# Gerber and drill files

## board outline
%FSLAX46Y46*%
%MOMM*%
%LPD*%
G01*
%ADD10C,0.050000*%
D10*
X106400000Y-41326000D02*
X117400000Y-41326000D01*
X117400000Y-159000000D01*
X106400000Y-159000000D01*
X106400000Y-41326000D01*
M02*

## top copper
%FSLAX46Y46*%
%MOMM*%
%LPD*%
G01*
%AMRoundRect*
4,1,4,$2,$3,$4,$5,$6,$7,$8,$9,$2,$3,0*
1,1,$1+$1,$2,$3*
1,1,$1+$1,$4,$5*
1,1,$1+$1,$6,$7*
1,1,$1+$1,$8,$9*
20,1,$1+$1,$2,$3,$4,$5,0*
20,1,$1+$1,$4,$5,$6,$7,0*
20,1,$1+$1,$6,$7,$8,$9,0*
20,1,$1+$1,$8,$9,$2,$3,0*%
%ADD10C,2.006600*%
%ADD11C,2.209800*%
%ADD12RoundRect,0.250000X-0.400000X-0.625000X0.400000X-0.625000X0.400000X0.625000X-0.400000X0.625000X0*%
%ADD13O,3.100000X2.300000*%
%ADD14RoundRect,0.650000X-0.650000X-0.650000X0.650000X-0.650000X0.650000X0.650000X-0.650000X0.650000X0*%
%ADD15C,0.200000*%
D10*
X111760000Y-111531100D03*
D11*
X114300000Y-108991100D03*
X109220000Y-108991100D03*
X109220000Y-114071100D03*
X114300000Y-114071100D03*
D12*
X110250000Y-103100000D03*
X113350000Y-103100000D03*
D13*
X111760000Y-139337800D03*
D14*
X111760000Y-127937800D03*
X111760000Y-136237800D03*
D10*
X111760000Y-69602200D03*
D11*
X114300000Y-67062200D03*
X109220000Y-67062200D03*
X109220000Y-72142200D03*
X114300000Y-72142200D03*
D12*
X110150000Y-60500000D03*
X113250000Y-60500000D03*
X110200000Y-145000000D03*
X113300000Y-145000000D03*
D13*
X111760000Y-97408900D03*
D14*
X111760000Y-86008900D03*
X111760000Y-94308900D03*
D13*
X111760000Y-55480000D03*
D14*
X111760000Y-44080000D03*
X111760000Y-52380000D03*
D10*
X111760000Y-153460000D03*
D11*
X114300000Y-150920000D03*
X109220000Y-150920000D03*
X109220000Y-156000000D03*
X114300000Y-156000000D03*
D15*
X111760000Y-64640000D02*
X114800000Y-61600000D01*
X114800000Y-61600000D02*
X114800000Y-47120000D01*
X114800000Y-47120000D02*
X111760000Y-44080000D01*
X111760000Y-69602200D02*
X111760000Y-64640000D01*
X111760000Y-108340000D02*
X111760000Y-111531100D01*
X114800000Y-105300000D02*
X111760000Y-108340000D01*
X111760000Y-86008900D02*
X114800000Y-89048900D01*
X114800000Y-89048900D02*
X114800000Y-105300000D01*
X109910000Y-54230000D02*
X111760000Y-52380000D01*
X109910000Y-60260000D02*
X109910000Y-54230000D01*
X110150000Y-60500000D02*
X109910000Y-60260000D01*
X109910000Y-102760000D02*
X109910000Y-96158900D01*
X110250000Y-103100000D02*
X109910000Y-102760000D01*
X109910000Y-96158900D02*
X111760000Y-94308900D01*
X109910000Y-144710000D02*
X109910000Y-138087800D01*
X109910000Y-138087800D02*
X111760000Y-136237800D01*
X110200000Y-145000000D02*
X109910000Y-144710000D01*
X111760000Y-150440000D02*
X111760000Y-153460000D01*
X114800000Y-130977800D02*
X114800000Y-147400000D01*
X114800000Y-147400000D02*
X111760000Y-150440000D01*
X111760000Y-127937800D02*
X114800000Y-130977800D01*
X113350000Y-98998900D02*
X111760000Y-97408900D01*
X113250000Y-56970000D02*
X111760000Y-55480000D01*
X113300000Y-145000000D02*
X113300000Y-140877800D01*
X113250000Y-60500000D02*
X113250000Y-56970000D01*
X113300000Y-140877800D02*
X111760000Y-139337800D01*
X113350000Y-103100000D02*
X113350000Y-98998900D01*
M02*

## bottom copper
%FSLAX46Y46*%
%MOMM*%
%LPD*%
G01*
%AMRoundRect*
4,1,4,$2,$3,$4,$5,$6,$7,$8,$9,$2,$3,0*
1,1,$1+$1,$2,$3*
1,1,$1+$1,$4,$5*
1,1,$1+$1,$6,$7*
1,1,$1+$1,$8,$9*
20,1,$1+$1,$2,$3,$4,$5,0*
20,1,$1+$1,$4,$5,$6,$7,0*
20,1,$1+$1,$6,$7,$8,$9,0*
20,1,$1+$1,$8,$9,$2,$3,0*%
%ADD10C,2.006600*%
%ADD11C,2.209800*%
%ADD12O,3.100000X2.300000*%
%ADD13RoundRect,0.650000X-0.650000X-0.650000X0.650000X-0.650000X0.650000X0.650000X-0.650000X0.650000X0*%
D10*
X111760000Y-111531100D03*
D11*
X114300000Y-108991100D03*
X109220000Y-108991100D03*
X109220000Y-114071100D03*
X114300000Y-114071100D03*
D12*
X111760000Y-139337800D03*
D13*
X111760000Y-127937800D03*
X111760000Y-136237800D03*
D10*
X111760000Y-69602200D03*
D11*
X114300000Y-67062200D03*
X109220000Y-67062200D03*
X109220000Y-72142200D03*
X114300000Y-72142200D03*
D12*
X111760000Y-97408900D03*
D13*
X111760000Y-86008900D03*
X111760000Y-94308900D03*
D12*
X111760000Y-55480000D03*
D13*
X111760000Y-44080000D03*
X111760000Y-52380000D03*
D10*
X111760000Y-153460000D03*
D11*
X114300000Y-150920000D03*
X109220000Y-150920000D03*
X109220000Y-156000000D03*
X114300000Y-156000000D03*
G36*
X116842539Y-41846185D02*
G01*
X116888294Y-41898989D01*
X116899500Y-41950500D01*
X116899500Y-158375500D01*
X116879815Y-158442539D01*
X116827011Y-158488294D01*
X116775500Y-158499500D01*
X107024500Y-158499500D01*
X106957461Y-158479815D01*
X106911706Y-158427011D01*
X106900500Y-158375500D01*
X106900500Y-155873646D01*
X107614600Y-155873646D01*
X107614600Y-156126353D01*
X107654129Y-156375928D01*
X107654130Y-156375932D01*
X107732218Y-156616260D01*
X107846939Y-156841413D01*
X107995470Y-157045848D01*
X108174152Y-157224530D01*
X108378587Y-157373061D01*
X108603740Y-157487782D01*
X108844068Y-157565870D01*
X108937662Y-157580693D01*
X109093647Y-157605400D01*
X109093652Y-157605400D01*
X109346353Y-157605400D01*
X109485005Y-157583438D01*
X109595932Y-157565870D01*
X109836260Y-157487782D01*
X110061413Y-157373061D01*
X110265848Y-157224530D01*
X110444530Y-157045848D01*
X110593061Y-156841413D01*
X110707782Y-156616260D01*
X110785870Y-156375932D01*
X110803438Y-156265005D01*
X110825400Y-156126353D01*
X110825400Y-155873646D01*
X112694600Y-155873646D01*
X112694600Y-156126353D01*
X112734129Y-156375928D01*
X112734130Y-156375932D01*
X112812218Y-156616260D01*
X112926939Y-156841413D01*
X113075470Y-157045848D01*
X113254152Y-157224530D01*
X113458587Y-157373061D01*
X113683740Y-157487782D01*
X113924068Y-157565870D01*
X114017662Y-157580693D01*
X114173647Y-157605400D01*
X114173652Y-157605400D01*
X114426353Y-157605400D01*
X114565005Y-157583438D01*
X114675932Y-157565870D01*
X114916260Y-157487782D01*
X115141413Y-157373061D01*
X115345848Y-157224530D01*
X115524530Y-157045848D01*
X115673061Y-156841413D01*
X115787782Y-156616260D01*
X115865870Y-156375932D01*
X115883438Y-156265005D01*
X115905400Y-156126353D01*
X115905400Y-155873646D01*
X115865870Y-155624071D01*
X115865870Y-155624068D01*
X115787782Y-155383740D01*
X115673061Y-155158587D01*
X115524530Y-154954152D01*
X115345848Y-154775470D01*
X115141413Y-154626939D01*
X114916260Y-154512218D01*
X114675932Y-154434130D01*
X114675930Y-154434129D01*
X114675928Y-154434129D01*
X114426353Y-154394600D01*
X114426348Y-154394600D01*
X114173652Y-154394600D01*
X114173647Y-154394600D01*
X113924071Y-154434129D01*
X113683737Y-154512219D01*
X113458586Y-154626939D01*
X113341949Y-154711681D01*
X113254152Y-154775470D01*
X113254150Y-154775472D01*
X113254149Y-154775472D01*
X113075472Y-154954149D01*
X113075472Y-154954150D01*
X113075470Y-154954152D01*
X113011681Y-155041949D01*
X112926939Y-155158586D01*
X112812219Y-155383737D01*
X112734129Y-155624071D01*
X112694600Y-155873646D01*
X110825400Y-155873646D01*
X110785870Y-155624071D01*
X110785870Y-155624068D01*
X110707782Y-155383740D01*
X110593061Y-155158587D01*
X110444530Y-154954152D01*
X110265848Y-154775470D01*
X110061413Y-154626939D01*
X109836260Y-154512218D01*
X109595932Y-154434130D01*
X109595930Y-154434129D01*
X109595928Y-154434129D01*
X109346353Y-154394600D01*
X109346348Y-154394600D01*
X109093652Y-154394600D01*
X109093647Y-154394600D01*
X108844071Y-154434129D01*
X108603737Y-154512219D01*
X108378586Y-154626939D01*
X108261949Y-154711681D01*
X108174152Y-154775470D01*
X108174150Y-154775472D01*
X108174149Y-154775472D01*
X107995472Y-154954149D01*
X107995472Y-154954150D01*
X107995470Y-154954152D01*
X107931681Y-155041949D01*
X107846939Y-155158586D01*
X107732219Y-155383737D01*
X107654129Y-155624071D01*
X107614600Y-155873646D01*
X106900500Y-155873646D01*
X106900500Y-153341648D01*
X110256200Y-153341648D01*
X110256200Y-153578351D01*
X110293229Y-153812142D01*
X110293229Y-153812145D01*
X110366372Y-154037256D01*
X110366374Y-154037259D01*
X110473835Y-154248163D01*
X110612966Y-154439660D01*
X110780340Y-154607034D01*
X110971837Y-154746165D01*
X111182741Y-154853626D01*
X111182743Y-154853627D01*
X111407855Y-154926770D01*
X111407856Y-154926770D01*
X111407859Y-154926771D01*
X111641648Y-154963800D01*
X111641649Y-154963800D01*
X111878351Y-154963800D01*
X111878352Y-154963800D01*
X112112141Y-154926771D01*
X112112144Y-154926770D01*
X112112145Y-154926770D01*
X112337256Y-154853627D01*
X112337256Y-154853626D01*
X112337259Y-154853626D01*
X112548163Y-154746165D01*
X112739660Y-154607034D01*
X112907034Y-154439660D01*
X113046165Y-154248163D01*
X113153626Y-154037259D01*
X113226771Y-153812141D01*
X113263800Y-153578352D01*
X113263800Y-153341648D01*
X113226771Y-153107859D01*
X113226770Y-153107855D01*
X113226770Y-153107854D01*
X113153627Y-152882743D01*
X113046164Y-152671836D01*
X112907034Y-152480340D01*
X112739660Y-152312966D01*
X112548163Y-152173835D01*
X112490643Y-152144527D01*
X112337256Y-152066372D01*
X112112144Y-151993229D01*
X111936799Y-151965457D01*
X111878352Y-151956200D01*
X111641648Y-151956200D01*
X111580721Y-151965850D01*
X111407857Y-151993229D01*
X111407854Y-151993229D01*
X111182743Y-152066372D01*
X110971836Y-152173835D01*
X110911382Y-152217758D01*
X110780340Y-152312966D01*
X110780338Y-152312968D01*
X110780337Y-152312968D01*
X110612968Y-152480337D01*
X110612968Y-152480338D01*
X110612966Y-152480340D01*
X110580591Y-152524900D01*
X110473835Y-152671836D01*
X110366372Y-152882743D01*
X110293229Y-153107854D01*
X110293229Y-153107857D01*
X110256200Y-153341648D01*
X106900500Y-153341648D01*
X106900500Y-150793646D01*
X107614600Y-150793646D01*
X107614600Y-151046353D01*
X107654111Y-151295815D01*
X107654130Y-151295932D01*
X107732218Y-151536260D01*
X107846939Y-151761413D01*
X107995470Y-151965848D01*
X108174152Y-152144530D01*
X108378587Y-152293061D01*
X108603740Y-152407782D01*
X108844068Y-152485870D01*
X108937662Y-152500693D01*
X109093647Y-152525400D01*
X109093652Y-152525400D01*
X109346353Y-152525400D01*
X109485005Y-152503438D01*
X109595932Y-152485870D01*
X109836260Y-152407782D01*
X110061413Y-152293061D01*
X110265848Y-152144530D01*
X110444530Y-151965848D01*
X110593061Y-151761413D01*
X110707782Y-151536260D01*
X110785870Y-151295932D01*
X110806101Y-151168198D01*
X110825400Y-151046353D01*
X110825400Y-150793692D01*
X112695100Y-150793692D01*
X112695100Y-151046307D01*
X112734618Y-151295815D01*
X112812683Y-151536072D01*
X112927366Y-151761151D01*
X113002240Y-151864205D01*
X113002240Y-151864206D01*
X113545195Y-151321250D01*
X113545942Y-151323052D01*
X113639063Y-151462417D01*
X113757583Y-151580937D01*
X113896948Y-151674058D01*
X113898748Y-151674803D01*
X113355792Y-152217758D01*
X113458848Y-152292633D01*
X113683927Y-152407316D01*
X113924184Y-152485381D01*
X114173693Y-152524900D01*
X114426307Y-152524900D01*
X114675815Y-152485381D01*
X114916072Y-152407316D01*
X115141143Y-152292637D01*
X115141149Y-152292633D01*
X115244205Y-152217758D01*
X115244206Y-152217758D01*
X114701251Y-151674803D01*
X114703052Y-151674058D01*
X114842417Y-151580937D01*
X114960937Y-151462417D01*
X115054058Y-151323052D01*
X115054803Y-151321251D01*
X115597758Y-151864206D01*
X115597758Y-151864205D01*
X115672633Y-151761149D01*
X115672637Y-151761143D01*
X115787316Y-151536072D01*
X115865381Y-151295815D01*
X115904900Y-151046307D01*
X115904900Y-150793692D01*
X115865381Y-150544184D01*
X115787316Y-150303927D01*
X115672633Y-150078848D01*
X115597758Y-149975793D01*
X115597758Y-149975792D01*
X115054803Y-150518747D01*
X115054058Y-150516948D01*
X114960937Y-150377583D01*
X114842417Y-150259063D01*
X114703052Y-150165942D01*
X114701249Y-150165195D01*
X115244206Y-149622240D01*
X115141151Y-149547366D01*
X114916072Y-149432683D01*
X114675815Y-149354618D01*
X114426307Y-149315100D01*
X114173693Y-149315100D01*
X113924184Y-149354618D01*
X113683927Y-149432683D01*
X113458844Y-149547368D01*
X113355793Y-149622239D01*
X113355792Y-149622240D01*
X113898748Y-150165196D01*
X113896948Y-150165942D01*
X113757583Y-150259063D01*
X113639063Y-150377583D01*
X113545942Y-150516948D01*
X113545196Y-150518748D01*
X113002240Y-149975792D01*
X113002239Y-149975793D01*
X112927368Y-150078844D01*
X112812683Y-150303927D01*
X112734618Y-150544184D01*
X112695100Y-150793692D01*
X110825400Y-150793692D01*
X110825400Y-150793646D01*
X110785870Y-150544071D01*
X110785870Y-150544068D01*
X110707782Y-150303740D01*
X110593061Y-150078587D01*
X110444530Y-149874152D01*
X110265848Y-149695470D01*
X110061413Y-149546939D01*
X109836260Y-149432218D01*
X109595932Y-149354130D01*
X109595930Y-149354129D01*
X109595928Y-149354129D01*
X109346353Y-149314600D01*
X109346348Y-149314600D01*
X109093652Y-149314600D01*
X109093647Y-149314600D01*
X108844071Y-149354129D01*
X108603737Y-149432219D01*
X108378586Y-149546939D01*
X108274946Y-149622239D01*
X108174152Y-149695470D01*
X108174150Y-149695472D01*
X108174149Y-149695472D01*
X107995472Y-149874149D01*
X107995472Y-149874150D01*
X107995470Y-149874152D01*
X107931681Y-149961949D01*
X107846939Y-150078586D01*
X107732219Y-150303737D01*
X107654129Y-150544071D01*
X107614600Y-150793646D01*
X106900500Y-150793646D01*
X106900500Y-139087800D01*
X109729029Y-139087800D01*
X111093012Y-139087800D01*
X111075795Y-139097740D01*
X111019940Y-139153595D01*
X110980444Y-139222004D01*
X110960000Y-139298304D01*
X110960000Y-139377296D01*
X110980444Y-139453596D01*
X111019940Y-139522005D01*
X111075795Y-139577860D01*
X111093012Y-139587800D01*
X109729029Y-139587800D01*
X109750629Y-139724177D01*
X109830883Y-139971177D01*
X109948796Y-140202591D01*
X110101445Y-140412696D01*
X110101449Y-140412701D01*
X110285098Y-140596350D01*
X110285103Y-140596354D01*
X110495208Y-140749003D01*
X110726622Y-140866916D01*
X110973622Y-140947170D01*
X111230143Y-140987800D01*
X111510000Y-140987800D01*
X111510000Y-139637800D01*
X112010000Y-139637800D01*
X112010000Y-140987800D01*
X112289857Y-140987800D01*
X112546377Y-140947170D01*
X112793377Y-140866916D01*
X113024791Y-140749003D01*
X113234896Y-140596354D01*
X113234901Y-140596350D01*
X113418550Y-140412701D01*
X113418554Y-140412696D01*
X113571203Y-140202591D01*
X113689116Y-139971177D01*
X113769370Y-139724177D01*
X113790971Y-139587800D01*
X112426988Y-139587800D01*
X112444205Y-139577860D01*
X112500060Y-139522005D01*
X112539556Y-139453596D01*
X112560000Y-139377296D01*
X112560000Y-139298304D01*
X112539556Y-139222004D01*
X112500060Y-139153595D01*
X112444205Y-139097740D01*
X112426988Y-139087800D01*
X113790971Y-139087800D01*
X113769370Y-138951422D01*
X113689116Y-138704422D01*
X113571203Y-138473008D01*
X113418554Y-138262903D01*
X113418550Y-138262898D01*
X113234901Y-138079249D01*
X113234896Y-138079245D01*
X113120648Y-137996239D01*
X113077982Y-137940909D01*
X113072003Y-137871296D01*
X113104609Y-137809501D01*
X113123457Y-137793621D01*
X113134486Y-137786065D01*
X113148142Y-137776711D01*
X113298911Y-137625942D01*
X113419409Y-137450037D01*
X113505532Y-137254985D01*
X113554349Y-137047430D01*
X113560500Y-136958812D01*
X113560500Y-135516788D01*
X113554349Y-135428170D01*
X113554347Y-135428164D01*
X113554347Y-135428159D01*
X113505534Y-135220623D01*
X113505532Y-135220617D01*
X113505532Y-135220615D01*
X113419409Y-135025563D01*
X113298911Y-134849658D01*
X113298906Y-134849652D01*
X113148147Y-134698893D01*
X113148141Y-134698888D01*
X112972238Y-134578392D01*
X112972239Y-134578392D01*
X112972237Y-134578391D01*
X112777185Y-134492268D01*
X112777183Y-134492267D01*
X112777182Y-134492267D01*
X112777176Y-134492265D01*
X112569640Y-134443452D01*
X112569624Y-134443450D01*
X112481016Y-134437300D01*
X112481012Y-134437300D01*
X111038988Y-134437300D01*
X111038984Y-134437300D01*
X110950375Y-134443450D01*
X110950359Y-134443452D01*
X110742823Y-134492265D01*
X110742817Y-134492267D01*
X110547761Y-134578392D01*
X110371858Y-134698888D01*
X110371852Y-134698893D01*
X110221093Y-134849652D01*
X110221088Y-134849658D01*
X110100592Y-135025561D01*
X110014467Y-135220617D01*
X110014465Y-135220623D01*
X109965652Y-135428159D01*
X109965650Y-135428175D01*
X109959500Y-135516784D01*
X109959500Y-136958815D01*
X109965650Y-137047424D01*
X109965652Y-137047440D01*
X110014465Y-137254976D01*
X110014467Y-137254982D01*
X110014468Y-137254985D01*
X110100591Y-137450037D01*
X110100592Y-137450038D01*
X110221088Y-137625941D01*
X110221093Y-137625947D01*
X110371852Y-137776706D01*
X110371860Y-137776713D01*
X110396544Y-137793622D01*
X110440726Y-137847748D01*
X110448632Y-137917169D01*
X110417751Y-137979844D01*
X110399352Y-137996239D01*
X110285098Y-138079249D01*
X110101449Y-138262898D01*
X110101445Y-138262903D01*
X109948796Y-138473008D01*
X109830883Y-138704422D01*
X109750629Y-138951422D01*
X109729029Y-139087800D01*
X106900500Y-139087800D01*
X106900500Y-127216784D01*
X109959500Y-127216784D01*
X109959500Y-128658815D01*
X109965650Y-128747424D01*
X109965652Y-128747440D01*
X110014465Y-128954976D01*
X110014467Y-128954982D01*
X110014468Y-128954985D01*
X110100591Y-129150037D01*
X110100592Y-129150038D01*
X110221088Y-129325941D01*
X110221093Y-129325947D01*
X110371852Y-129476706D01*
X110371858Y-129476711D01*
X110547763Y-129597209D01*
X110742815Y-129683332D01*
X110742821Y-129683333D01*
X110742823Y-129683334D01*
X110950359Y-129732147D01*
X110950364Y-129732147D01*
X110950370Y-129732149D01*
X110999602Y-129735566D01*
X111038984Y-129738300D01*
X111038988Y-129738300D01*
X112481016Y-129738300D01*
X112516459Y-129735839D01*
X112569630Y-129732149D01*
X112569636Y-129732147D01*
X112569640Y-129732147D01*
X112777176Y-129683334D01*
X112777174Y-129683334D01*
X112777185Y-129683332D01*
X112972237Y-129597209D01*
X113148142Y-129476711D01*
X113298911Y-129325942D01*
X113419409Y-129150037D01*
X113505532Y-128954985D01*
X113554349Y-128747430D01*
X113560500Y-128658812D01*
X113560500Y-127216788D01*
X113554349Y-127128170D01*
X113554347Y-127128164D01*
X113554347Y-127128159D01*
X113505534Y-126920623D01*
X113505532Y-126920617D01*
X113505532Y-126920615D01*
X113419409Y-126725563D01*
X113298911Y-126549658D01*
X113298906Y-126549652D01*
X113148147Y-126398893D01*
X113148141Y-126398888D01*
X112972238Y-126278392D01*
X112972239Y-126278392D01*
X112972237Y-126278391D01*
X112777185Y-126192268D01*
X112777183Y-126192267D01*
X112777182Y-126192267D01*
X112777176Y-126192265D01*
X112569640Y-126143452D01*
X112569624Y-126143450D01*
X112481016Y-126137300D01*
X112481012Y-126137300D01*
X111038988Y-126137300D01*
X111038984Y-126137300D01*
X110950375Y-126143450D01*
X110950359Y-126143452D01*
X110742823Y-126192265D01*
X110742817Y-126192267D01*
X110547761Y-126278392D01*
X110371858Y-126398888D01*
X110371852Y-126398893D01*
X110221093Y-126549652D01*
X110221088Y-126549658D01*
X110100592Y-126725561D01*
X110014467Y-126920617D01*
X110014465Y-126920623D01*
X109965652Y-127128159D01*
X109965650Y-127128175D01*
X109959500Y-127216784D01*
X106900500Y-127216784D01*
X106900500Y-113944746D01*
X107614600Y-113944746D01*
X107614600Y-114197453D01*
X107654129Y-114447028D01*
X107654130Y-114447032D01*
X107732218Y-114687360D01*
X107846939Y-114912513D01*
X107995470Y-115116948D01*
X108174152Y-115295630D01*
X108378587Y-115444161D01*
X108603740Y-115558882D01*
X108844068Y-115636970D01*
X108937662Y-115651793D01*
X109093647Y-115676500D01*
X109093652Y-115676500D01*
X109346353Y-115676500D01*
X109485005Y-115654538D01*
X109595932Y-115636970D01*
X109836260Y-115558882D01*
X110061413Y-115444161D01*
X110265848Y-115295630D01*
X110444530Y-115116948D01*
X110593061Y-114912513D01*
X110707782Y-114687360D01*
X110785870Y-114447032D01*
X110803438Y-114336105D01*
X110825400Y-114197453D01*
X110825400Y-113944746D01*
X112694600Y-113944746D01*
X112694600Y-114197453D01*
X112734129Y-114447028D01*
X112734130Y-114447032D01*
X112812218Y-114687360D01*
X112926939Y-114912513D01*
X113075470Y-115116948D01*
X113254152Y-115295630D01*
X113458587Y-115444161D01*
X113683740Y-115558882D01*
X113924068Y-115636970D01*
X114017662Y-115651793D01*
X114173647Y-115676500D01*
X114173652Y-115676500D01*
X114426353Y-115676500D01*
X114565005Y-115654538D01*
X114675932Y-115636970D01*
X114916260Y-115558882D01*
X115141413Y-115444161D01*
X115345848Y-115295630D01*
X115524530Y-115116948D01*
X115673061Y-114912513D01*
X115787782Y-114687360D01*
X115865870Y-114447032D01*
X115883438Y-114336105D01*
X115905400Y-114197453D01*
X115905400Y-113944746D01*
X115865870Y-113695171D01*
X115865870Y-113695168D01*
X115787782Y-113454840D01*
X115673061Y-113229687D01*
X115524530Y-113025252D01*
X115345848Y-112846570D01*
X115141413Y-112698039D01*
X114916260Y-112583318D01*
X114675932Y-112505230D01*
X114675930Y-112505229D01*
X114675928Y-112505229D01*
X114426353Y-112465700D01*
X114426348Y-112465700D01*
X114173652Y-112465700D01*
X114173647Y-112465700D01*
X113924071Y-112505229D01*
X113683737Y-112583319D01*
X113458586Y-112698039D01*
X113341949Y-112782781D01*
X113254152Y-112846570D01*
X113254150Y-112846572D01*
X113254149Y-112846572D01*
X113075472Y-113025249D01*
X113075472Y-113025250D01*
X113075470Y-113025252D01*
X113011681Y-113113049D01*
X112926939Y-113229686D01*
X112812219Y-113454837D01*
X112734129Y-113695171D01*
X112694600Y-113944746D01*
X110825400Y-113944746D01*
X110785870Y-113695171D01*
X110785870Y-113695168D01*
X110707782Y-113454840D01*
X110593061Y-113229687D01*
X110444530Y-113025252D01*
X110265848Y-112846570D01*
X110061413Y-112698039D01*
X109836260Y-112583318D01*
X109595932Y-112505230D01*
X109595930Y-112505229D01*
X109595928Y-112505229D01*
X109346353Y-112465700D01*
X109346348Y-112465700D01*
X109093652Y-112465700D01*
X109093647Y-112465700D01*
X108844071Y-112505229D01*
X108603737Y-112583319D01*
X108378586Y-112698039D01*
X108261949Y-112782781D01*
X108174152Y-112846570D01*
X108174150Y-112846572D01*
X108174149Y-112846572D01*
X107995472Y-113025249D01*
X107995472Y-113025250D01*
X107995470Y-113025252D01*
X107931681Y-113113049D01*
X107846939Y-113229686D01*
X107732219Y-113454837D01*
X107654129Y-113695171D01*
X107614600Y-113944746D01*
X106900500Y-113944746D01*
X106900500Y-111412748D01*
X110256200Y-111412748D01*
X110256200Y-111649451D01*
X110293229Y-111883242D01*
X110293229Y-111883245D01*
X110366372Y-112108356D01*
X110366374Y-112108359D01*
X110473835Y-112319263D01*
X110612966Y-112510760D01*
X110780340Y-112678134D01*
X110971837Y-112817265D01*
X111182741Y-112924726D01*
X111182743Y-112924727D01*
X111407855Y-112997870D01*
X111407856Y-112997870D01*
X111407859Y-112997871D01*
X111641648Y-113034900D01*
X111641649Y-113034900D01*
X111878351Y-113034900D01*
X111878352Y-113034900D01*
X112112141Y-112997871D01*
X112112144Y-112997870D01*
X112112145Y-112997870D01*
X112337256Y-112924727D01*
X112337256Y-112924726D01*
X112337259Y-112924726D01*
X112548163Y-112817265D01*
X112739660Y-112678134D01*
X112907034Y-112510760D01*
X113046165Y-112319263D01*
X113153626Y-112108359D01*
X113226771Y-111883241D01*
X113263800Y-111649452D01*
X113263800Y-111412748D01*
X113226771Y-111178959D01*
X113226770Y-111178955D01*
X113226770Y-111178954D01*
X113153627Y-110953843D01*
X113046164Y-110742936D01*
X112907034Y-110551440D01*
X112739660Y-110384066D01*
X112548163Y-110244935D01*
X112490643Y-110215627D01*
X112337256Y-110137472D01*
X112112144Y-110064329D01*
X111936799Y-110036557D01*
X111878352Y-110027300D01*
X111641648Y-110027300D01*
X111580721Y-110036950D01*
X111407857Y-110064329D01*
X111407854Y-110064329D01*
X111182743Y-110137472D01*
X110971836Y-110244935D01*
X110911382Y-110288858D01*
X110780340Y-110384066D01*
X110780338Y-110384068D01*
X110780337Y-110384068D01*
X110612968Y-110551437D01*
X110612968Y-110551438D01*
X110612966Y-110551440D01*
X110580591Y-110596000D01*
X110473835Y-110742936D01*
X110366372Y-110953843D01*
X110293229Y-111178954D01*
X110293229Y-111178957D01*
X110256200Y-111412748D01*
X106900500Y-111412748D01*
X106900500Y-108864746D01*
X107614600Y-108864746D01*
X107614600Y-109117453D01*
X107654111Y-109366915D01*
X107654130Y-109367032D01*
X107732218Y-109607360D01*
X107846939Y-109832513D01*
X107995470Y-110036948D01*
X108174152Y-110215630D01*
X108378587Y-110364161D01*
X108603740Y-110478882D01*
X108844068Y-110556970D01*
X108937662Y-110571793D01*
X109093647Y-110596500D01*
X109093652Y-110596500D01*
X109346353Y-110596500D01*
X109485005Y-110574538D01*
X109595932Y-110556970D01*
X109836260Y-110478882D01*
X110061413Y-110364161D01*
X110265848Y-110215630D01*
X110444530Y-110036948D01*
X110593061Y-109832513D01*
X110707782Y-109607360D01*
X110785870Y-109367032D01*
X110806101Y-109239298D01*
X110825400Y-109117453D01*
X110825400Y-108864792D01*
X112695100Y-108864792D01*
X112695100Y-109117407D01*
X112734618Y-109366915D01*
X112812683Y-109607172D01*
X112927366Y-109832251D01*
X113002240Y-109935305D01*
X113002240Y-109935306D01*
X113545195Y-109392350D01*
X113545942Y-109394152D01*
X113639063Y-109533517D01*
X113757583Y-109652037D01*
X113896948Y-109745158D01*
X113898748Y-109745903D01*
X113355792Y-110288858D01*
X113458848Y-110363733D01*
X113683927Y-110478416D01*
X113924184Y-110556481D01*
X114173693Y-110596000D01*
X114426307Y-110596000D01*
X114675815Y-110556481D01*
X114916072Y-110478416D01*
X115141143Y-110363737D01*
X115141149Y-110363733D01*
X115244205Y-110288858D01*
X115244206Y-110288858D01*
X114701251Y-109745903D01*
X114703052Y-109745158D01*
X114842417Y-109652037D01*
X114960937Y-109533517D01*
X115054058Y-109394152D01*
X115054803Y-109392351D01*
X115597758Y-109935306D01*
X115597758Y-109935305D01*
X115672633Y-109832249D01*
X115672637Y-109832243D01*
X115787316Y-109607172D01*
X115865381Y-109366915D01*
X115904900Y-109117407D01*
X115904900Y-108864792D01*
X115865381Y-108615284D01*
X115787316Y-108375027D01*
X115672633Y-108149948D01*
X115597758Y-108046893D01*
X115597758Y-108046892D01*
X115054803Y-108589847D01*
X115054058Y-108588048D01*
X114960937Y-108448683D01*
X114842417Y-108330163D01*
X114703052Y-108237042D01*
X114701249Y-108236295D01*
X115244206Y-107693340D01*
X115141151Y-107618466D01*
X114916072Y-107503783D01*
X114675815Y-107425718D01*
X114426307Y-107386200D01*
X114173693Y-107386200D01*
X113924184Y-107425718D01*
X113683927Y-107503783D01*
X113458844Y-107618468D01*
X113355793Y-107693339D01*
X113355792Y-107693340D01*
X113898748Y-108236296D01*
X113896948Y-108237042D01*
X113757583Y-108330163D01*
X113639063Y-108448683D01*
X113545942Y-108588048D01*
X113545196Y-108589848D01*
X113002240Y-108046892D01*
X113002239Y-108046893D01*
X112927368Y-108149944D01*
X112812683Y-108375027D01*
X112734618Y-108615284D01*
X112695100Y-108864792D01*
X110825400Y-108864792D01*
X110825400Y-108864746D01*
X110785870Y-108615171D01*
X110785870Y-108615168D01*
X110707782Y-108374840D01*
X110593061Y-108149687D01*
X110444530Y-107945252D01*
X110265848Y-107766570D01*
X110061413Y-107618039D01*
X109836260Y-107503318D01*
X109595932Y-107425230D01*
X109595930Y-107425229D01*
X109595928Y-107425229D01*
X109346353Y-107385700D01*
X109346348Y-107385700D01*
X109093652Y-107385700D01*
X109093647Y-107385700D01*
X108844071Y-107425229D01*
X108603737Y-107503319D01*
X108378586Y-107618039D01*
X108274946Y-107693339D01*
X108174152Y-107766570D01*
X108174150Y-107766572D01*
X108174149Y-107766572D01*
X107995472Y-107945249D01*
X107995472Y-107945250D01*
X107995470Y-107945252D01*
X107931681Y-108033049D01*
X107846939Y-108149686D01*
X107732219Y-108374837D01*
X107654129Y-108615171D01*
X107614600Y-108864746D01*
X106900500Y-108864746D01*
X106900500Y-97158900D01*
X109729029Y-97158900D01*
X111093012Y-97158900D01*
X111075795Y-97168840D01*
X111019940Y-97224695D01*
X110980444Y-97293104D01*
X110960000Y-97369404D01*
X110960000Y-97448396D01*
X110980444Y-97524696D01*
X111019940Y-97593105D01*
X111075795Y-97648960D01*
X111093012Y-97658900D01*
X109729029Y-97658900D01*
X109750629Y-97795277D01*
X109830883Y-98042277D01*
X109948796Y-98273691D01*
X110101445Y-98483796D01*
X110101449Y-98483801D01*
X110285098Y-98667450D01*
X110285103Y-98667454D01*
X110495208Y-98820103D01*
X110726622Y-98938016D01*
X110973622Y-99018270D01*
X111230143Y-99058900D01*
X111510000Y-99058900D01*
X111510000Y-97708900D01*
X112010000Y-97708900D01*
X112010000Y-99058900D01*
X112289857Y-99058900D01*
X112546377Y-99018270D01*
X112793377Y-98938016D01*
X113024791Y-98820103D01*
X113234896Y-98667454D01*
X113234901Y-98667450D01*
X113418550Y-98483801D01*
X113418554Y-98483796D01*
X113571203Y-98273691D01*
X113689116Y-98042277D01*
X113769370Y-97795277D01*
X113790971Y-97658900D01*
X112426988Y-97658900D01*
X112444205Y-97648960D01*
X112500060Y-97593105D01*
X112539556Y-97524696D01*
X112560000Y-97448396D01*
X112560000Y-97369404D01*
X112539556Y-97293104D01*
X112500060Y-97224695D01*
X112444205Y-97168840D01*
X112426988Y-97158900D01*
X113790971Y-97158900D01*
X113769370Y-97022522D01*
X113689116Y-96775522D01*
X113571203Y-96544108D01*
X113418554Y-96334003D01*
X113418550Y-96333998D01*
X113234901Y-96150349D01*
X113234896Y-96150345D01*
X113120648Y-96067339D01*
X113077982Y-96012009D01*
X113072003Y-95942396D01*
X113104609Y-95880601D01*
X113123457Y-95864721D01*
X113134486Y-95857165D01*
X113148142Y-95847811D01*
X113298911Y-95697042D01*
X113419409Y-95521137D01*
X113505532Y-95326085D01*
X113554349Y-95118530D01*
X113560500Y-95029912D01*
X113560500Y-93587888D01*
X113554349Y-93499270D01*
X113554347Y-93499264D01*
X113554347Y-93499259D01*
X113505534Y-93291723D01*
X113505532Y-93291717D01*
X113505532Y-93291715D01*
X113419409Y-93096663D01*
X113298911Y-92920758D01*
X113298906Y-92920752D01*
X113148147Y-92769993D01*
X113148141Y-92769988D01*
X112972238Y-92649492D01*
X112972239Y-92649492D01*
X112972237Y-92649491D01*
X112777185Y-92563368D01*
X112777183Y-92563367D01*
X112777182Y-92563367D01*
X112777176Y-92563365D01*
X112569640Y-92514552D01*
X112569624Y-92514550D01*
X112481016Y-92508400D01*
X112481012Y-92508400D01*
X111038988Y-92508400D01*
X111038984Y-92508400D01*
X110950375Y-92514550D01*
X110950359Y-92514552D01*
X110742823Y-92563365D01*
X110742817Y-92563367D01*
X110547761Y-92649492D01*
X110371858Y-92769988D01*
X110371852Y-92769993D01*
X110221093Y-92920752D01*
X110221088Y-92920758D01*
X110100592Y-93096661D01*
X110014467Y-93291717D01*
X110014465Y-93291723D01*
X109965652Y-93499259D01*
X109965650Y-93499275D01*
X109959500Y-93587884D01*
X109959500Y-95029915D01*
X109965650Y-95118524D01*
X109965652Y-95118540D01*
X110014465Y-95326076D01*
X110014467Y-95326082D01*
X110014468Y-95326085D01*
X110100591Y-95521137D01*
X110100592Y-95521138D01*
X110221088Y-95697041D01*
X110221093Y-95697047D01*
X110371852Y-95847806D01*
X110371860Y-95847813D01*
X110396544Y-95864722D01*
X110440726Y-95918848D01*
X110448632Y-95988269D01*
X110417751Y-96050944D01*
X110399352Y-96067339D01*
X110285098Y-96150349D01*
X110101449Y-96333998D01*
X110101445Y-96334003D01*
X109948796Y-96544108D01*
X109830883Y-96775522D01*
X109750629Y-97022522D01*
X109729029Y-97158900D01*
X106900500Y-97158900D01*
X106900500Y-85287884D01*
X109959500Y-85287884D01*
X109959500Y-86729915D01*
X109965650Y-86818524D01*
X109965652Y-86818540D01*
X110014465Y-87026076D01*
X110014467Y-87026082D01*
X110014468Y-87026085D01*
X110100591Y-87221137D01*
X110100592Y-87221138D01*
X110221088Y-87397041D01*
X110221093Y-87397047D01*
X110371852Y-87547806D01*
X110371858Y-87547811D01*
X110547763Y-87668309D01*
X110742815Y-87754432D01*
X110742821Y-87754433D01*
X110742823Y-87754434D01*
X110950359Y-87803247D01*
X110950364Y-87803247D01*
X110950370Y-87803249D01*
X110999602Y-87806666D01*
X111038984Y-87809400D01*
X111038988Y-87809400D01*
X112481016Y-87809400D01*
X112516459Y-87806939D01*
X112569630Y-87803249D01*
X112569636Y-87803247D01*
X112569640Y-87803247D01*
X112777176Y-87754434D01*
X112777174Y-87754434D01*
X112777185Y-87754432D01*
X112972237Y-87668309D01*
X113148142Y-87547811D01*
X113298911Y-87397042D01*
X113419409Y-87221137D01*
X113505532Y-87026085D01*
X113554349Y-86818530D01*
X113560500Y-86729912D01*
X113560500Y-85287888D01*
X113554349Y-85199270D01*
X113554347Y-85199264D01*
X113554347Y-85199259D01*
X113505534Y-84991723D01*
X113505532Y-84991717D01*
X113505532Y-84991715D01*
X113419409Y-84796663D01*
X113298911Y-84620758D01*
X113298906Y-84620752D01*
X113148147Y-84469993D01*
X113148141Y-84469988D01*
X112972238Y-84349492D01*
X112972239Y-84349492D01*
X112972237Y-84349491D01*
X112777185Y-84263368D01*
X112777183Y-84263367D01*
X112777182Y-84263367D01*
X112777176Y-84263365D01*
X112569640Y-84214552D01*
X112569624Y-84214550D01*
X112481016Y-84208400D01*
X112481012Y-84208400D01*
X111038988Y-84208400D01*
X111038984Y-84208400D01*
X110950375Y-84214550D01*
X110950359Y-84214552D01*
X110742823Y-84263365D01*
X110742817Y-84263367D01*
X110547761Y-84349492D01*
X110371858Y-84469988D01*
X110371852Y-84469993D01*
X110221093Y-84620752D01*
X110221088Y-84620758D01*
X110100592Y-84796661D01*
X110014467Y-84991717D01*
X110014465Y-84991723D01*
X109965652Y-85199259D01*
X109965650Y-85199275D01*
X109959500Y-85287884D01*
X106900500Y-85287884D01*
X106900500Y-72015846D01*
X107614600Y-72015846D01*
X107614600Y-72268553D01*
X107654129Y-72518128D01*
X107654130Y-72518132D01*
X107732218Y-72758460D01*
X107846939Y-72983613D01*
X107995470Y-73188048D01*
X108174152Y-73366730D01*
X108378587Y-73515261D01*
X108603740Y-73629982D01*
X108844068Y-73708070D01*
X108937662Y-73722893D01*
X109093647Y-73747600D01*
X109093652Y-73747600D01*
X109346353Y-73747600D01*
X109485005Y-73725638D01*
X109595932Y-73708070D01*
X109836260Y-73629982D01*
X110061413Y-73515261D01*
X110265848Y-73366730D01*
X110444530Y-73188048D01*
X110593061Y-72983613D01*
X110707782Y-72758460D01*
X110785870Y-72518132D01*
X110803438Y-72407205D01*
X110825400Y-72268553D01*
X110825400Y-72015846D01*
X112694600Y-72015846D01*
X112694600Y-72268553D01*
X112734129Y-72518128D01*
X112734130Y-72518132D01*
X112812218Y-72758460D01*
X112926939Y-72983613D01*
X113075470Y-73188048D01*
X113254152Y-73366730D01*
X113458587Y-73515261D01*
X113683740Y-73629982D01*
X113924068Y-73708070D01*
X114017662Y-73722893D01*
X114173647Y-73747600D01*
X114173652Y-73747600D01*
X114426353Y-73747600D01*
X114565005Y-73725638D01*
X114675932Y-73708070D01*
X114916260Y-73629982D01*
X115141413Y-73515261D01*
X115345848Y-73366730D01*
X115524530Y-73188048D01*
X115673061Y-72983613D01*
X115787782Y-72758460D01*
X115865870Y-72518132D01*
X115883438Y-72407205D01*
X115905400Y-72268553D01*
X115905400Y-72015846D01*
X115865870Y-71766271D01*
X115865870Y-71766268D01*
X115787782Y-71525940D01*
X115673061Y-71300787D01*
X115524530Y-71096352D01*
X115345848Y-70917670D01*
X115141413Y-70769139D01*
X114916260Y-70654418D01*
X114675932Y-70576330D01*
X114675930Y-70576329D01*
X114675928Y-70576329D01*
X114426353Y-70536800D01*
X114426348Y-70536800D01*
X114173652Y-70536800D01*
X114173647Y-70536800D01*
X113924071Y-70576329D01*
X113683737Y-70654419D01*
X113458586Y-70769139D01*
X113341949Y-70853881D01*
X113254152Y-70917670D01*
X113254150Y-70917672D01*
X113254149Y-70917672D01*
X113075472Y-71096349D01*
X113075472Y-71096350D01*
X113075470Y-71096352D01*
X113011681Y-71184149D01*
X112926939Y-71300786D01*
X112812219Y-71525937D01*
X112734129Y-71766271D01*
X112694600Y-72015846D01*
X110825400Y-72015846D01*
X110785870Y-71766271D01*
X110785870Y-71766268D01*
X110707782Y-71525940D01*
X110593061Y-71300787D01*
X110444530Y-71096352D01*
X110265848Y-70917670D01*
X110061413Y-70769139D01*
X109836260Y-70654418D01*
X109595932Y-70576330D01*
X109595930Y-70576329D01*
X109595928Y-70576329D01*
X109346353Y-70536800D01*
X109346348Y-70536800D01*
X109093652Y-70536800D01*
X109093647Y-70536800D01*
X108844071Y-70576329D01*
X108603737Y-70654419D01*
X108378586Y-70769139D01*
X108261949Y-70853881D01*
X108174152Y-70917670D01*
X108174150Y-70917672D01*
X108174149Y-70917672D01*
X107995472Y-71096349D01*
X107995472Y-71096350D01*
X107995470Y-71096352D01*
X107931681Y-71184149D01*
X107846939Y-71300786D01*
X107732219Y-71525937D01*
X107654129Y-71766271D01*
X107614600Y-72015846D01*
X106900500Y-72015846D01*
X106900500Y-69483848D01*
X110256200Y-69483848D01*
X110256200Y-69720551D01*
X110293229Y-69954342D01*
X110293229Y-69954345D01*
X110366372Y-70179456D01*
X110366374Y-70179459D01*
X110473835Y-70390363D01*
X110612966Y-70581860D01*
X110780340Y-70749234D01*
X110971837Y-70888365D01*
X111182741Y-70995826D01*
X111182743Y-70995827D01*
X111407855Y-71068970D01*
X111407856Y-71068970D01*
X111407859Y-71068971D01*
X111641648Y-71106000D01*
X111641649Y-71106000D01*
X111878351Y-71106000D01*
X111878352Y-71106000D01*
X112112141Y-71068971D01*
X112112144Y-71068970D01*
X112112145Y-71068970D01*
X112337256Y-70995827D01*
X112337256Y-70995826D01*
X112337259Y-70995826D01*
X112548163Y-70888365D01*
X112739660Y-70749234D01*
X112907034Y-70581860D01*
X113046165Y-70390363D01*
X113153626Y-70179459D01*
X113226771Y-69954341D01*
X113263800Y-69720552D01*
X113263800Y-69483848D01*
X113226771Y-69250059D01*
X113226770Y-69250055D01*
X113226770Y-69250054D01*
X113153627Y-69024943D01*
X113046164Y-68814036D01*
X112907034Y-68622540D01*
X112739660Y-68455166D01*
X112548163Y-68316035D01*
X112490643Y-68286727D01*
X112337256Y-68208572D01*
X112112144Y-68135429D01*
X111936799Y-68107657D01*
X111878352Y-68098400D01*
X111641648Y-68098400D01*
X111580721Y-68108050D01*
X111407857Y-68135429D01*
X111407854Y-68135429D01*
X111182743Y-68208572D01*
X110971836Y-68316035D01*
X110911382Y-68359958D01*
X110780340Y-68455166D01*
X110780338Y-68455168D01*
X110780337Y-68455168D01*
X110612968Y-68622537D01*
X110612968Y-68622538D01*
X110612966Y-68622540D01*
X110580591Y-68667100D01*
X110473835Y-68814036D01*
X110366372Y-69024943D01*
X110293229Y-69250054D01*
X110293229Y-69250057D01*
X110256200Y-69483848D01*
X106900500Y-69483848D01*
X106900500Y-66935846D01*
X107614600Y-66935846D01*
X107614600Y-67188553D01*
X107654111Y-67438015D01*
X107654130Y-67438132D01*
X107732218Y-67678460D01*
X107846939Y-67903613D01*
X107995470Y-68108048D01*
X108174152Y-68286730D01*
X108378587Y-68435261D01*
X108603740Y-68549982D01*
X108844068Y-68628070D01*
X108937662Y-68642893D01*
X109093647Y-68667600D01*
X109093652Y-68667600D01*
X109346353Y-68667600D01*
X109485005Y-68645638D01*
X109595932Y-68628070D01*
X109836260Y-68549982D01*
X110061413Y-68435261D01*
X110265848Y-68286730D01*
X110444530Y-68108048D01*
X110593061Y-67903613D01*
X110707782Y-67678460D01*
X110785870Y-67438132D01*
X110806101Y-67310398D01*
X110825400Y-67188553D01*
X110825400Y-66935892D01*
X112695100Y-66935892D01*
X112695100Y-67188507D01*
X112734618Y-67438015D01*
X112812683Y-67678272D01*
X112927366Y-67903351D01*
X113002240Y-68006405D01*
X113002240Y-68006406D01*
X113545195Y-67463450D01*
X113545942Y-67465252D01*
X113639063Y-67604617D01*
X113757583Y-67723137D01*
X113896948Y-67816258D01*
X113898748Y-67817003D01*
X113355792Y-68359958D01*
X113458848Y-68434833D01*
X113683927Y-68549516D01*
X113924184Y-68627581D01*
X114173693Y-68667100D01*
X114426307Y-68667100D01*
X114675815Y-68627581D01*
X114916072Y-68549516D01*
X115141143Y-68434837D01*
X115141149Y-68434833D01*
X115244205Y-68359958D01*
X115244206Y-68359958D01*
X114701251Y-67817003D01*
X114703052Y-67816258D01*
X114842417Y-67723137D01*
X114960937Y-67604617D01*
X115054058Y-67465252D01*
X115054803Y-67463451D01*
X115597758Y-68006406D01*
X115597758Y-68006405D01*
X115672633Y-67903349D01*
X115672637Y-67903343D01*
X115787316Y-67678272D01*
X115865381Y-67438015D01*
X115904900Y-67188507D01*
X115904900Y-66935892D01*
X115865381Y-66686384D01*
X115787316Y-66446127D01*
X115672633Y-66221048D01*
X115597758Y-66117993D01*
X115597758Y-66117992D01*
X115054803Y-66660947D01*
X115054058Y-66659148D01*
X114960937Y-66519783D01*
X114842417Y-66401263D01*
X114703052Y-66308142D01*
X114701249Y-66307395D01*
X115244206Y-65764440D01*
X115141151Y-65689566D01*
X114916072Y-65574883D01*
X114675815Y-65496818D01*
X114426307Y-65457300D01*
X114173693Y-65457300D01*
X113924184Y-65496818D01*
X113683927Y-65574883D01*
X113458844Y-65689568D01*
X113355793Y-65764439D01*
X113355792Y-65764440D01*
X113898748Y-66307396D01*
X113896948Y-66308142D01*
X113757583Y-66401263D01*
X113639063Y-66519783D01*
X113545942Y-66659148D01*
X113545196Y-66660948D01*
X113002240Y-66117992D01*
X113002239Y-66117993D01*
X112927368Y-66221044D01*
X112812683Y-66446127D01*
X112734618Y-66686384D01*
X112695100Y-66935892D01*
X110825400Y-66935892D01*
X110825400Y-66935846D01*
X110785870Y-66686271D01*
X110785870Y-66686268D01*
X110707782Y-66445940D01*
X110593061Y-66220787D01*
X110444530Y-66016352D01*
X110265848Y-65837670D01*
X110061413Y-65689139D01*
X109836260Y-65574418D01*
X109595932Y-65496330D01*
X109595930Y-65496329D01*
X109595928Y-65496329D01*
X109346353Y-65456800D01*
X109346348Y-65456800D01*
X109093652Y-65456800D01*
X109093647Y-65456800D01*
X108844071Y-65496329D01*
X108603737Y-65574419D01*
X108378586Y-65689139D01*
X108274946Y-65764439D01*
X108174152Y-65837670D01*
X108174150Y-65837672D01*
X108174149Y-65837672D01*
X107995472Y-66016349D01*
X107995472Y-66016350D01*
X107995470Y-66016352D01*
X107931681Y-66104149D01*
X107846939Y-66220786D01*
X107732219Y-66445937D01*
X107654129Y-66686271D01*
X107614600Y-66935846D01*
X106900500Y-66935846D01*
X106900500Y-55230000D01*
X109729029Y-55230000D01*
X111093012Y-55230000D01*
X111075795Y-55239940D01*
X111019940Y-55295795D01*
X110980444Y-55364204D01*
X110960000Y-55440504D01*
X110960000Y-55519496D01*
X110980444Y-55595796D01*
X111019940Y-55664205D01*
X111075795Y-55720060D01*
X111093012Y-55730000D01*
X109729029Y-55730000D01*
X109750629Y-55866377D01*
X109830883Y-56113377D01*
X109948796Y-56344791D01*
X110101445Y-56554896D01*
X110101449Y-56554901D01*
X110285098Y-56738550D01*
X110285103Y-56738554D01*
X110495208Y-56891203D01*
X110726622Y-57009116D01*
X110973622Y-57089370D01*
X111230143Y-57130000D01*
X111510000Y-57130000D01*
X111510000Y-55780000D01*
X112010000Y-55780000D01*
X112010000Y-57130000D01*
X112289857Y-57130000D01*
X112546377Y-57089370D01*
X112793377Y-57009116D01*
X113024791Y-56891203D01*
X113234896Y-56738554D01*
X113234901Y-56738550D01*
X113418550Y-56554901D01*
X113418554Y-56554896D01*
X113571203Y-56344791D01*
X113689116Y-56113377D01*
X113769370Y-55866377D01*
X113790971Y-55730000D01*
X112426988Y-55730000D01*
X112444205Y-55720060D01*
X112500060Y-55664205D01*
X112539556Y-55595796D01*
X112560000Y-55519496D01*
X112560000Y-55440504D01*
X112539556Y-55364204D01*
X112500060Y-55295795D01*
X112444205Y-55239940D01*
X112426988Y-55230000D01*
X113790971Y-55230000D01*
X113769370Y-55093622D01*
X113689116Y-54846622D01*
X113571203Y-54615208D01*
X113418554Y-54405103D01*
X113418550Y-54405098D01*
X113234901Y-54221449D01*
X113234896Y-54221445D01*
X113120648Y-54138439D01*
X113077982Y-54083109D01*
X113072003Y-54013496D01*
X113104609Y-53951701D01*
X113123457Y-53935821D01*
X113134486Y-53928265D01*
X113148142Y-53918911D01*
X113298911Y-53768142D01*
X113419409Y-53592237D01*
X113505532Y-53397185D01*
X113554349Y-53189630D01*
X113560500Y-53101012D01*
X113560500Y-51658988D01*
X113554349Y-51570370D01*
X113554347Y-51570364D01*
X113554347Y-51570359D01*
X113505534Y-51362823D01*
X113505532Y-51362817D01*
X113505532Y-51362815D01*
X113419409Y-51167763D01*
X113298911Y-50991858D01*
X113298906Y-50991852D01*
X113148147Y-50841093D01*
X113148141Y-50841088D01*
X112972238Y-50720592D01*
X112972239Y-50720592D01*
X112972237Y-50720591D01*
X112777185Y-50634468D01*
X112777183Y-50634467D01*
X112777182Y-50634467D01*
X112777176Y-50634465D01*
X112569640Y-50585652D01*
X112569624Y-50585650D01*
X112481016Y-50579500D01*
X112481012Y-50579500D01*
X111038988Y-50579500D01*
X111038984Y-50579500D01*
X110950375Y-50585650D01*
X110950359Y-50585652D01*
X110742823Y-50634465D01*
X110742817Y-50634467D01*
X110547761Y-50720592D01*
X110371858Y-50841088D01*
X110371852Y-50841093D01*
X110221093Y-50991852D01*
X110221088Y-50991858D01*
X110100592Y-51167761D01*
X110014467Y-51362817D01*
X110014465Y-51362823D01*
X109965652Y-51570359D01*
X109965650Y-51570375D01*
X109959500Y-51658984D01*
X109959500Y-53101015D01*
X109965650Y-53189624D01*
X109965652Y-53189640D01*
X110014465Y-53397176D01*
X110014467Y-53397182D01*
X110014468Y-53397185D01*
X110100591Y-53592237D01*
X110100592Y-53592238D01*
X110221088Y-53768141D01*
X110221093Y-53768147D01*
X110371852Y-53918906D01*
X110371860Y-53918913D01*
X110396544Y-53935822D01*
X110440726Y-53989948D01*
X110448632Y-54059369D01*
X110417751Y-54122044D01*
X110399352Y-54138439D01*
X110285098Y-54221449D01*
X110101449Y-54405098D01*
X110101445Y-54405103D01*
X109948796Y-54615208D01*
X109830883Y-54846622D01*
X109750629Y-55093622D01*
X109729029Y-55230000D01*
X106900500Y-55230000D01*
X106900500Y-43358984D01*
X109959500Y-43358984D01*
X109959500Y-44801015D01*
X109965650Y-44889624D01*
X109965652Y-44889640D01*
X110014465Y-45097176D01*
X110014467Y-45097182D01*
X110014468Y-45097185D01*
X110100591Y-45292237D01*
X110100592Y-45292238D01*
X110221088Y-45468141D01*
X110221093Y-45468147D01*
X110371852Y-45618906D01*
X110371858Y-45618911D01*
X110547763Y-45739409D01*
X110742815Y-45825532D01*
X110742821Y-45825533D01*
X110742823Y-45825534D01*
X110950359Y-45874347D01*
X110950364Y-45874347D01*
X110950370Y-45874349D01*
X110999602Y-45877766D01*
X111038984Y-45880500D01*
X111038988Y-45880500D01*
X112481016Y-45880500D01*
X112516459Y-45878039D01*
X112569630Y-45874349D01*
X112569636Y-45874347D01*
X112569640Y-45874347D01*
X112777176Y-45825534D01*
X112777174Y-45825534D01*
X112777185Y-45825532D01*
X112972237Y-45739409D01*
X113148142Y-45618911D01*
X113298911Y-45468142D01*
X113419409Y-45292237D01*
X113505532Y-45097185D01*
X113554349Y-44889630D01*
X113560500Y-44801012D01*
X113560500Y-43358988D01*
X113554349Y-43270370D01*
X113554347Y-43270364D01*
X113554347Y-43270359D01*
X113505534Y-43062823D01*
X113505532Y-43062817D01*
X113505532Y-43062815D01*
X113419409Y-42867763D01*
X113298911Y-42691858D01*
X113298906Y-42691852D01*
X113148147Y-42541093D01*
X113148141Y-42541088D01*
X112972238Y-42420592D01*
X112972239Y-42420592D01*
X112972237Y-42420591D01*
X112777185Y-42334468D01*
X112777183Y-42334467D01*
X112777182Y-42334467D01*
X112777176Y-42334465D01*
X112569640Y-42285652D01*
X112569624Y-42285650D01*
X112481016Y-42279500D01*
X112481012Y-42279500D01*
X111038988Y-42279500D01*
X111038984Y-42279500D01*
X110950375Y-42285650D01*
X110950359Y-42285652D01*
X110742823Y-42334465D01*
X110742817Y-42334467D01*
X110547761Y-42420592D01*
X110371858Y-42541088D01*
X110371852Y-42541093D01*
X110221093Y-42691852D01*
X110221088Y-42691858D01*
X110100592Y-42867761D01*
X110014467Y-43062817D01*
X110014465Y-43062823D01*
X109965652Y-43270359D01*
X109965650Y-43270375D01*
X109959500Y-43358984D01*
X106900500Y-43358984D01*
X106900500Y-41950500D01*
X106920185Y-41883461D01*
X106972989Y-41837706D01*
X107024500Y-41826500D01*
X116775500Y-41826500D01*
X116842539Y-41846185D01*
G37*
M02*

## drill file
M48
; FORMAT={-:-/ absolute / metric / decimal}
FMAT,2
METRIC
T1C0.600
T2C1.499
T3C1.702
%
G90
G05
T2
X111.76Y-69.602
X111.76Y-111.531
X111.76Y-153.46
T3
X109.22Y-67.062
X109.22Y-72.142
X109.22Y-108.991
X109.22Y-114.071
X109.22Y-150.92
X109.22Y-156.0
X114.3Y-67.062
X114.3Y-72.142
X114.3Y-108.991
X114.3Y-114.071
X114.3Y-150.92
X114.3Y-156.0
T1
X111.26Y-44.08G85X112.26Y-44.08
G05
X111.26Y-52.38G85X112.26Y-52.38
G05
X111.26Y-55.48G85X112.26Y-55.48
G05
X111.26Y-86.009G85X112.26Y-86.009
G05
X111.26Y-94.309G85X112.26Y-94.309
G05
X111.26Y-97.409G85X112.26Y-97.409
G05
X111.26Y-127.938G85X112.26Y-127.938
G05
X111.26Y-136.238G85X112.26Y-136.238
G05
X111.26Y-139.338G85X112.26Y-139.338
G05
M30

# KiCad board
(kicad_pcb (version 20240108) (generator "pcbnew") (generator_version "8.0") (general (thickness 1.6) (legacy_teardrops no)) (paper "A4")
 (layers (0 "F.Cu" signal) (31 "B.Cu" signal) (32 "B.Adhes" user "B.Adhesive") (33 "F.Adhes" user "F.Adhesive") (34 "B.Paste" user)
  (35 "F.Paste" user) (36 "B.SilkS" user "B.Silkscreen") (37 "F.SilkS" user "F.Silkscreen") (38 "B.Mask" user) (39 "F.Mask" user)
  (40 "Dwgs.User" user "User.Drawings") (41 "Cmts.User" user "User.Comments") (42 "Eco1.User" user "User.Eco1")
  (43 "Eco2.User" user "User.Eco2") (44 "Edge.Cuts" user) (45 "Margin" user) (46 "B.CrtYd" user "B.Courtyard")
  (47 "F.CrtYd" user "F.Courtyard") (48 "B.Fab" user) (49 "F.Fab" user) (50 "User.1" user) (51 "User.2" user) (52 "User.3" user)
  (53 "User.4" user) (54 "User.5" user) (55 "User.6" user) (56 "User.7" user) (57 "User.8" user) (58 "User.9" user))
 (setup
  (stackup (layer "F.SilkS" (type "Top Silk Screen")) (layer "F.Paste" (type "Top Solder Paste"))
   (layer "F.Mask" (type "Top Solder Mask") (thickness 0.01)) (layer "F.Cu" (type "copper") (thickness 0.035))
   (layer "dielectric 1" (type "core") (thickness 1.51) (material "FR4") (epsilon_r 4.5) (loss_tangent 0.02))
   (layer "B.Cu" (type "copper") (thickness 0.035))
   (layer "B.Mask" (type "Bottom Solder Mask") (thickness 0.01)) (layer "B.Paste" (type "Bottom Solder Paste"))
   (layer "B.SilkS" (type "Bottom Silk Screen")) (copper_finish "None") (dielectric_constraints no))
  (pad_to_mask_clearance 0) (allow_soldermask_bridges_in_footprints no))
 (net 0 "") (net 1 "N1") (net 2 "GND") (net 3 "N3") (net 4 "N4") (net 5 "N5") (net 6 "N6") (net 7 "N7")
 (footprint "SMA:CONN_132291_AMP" (layer "F.Cu") (at 111.76 111.5311 -90)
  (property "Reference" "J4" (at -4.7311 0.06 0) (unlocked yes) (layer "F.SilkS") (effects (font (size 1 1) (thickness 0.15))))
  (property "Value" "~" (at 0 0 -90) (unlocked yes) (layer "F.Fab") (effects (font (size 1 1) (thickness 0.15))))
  (pad "1" thru_hole circle (at 0 0 270) (size 2.0066 2.0066) (drill 1.4986) (layers "*.Cu" "*.Mask") (remove_unused_layers no) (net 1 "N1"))
  (pad "2" thru_hole circle (at -2.54 -2.54 270) (size 2.2098 2.2098) (drill 1.7018) (layers "*.Cu" "*.Mask") (remove_unused_layers no)
   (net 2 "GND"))
  (pad "3" thru_hole circle (at -2.54 2.54 270) (size 2.2098 2.2098) (drill 1.7018) (layers "*.Cu" "*.Mask") (remove_unused_layers no))
  (pad "4" thru_hole circle (at 2.54 2.54 270) (size 2.2098 2.2098) (drill 1.7018) (layers "*.Cu" "*.Mask") (remove_unused_layers no))
  (pad "5" thru_hole circle (at 2.54 -2.54 270) (size 2.2098 2.2098) (drill 1.7018) (layers "*.Cu" "*.Mask") (remove_unused_layers no)))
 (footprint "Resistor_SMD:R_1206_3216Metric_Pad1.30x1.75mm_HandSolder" (layer "F.Cu") (at 111.8 103.1)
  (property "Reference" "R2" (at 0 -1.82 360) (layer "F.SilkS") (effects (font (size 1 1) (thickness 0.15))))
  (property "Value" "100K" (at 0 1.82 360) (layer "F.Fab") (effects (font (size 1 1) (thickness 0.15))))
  (pad "1" smd roundrect (at -1.55 0) (size 1.3 1.75) (layers "F.Cu" "F.Paste" "F.Mask") (roundrect_rratio 0.192308) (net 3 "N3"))
  (pad "2" smd roundrect (at 1.55 0) (size 1.3 1.75) (layers "F.Cu" "F.Paste" "F.Mask") (roundrect_rratio 0.192308) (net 2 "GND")))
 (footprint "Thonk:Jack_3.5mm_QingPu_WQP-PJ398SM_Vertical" (layer "F.Cu") (at 111.76 132.8578)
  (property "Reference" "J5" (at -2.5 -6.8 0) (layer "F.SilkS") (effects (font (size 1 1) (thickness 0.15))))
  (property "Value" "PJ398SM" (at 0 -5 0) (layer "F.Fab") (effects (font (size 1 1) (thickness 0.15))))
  (pad "S" thru_hole oval (at 0 6.48) (size 3.1 2.3) (drill oval 1.6 0.6) (layers "*.Cu" "*.Mask") (remove_unused_layers no) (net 2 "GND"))
  (pad "T" thru_hole roundrect (at 0 -4.92) (size 2.6 2.6) (drill oval 1.6 0.6) (layers "*.Cu" "*.Mask") (remove_unused_layers no)
   (roundrect_rratio 0.25) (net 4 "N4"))
  (pad "TN" thru_hole roundrect (at 0 3.38) (size 2.6 2.6) (drill oval 1.6 0.6) (layers "*.Cu" "*.Mask") (remove_unused_layers no)
   (roundrect_rratio 0.25) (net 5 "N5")))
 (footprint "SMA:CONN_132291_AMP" (layer "F.Cu") (at 111.76 69.6022 -90)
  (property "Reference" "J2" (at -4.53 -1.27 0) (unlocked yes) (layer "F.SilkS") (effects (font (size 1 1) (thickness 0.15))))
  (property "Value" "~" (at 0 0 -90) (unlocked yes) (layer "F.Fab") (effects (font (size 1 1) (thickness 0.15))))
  (pad "1" thru_hole circle (at 0 0 270) (size 2.0066 2.0066) (drill 1.4986) (layers "*.Cu" "*.Mask") (remove_unused_layers no) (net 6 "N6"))
  (pad "2" thru_hole circle (at -2.54 -2.54 270) (size 2.2098 2.2098) (drill 1.7018) (layers "*.Cu" "*.Mask") (remove_unused_layers no)
   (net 2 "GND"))
  (pad "3" thru_hole circle (at -2.54 2.54 270) (size 2.2098 2.2098) (drill 1.7018) (layers "*.Cu" "*.Mask") (remove_unused_layers no))
  (pad "4" thru_hole circle (at 2.54 2.54 270) (size 2.2098 2.2098) (drill 1.7018) (layers "*.Cu" "*.Mask") (remove_unused_layers no))
  (pad "5" thru_hole circle (at 2.54 -2.54 270) (size 2.2098 2.2098) (drill 1.7018) (layers "*.Cu" "*.Mask") (remove_unused_layers no)))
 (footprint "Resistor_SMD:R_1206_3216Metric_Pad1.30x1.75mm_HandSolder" (layer "F.Cu") (at 111.7 60.5)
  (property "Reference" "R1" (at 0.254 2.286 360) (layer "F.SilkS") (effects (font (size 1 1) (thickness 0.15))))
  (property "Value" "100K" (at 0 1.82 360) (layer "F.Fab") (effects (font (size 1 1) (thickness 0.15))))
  (pad "1" smd roundrect (at -1.55 0) (size 1.3 1.75) (layers "F.Cu" "F.Paste" "F.Mask") (roundrect_rratio 0.192308) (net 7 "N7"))
  (pad "2" smd roundrect (at 1.55 0) (size 1.3 1.75) (layers "F.Cu" "F.Paste" "F.Mask") (roundrect_rratio 0.192308) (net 2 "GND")))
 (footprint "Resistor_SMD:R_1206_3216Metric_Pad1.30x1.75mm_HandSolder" (layer "F.Cu") (at 111.75 145)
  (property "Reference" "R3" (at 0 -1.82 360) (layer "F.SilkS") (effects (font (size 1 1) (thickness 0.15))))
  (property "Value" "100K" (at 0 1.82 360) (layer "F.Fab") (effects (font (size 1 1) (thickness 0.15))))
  (pad "1" smd roundrect (at -1.55 0) (size 1.3 1.75) (layers "F.Cu" "F.Paste" "F.Mask") (roundrect_rratio 0.192308) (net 5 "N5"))
  (pad "2" smd roundrect (at 1.55 0) (size 1.3 1.75) (layers "F.Cu" "F.Paste" "F.Mask") (roundrect_rratio 0.192308) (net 2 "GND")))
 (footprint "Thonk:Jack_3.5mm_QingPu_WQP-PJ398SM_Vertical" (layer "F.Cu") (at 111.76 90.9289)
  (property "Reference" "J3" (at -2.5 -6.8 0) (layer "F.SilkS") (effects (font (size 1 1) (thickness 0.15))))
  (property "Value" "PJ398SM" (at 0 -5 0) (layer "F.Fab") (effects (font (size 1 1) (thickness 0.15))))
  (pad "S" thru_hole oval (at 0 6.48) (size 3.1 2.3) (drill oval 1.6 0.6) (layers "*.Cu" "*.Mask") (remove_unused_layers no) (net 2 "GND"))
  (pad "T" thru_hole roundrect (at 0 -4.92) (size 2.6 2.6) (drill oval 1.6 0.6) (layers "*.Cu" "*.Mask") (remove_unused_layers no)
   (roundrect_rratio 0.25) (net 1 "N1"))
  (pad "TN" thru_hole roundrect (at 0 3.38) (size 2.6 2.6) (drill oval 1.6 0.6) (layers "*.Cu" "*.Mask") (remove_unused_layers no)
   (roundrect_rratio 0.25) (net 3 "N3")))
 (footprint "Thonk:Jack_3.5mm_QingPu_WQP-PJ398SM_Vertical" (layer "F.Cu") (at 111.76 49)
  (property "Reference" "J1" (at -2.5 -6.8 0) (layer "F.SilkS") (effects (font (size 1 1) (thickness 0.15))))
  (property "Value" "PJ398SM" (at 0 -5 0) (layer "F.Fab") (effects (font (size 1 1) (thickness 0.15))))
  (pad "S" thru_hole oval (at 0 6.48) (size 3.1 2.3) (drill oval 1.6 0.6) (layers "*.Cu" "*.Mask") (remove_unused_layers no) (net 2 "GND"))
  (pad "T" thru_hole roundrect (at 0 -4.92) (size 2.6 2.6) (drill oval 1.6 0.6) (layers "*.Cu" "*.Mask") (remove_unused_layers no)
   (roundrect_rratio 0.25) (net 6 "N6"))
  (pad "TN" thru_hole roundrect (at 0 3.38) (size 2.6 2.6) (drill oval 1.6 0.6) (layers "*.Cu" "*.Mask") (remove_unused_layers no)
   (roundrect_rratio 0.25) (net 7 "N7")))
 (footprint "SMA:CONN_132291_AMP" (layer "F.Cu") (at 111.76 153.46 -90)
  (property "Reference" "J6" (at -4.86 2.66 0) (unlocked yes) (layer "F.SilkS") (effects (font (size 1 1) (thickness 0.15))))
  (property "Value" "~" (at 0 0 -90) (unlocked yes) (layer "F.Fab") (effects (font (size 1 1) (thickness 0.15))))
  (pad "1" thru_hole circle (at 0 0 270) (size 2.0066 2.0066) (drill 1.4986) (layers "*.Cu" "*.Mask") (remove_unused_layers no) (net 4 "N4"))
  (pad "2" thru_hole circle (at -2.54 -2.54 270) (size 2.2098 2.2098) (drill 1.7018) (layers "*.Cu" "*.Mask") (remove_unused_layers no)
   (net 2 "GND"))
  (pad "3" thru_hole circle (at -2.54 2.54 270) (size 2.2098 2.2098) (drill 1.7018) (layers "*.Cu" "*.Mask") (remove_unused_layers no))
  (pad "4" thru_hole circle (at 2.54 2.54 270) (size 2.2098 2.2098) (drill 1.7018) (layers "*.Cu" "*.Mask") (remove_unused_layers no))
  (pad "5" thru_hole circle (at 2.54 -2.54 270) (size 2.2098 2.2098) (drill 1.7018) (layers "*.Cu" "*.Mask") (remove_unused_layers no)))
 (gr_rect (start 106.4 41.326) (end 117.4 159) (stroke (width 0.05) (type default)) (fill none) (layer "Edge.Cuts"))
 (segment (start 111.76 64.64) (end 114.8 61.6) (width 0.2) (layer "F.Cu") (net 6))
 (segment (start 114.8 61.6) (end 114.8 47.12) (width 0.2) (layer "F.Cu") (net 6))
 (segment (start 114.8 47.12) (end 111.76 44.08) (width 0.2) (layer "F.Cu") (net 6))
 (segment (start 111.76 69.6022) (end 111.76 64.64) (width 0.2) (layer "F.Cu") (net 6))
 (segment (start 111.76 108.34) (end 111.76 111.5311) (width 0.2) (layer "F.Cu") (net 1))
 (segment (start 114.8 105.3) (end 111.76 108.34) (width 0.2) (layer "F.Cu") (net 1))
 (segment (start 111.76 86.0089) (end 114.8 89.0489) (width 0.2) (layer "F.Cu") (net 1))
 (segment (start 114.8 89.0489) (end 114.8 105.3) (width 0.2) (layer "F.Cu") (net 1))
 (segment (start 109.91 54.23) (end 111.76 52.38) (width 0.2) (layer "F.Cu") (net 7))
 (segment (start 109.91 60.26) (end 109.91 54.23) (width 0.2) (layer "F.Cu") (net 7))
 (segment (start 110.15 60.5) (end 109.91 60.26) (width 0.2) (layer "F.Cu") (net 7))
 (segment (start 109.91 102.76) (end 109.91 96.1589) (width 0.2) (layer "F.Cu") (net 3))
 (segment (start 110.25 103.1) (end 109.91 102.76) (width 0.2) (layer "F.Cu") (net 3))
 (segment (start 109.91 96.1589) (end 111.76 94.3089) (width 0.2) (layer "F.Cu") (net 3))
 (segment (start 109.91 144.71) (end 109.91 138.0878) (width 0.2) (layer "F.Cu") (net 5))
 (segment (start 109.91 138.0878) (end 111.76 136.2378) (width 0.2) (layer "F.Cu") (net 5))
 (segment (start 110.2 145) (end 109.91 144.71) (width 0.2) (layer "F.Cu") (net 5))
 (segment (start 111.76 150.44) (end 111.76 153.46) (width 0.2) (layer "F.Cu") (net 4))
 (segment (start 114.8 130.9778) (end 114.8 147.4) (width 0.2) (layer "F.Cu") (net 4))
 (segment (start 114.8 147.4) (end 111.76 150.44) (width 0.2) (layer "F.Cu") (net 4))
 (segment (start 111.76 127.9378) (end 114.8 130.9778) (width 0.2) (layer "F.Cu") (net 4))
 (segment (start 113.35 98.9989) (end 111.76 97.4089) (width 0.2) (layer "F.Cu") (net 2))
 (segment (start 113.25 56.97) (end 111.76 55.48) (width 0.2) (layer "F.Cu") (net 2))
 (segment (start 113.3 145) (end 113.3 140.8778) (width 0.2) (layer "F.Cu") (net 2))
 (segment (start 113.25 60.5) (end 113.25 56.97) (width 0.2) (layer "F.Cu") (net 2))
 (segment (start 113.3 140.8778) (end 111.76 139.3378) (width 0.2) (layer "F.Cu") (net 2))
 (segment (start 113.35 103.1) (end 113.35 98.9989) (width 0.2) (layer "F.Cu") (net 2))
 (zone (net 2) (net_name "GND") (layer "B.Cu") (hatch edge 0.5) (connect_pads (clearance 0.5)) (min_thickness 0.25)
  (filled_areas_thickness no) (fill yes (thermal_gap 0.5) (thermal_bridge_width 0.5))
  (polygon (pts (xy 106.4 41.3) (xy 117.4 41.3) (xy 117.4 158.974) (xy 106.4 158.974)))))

